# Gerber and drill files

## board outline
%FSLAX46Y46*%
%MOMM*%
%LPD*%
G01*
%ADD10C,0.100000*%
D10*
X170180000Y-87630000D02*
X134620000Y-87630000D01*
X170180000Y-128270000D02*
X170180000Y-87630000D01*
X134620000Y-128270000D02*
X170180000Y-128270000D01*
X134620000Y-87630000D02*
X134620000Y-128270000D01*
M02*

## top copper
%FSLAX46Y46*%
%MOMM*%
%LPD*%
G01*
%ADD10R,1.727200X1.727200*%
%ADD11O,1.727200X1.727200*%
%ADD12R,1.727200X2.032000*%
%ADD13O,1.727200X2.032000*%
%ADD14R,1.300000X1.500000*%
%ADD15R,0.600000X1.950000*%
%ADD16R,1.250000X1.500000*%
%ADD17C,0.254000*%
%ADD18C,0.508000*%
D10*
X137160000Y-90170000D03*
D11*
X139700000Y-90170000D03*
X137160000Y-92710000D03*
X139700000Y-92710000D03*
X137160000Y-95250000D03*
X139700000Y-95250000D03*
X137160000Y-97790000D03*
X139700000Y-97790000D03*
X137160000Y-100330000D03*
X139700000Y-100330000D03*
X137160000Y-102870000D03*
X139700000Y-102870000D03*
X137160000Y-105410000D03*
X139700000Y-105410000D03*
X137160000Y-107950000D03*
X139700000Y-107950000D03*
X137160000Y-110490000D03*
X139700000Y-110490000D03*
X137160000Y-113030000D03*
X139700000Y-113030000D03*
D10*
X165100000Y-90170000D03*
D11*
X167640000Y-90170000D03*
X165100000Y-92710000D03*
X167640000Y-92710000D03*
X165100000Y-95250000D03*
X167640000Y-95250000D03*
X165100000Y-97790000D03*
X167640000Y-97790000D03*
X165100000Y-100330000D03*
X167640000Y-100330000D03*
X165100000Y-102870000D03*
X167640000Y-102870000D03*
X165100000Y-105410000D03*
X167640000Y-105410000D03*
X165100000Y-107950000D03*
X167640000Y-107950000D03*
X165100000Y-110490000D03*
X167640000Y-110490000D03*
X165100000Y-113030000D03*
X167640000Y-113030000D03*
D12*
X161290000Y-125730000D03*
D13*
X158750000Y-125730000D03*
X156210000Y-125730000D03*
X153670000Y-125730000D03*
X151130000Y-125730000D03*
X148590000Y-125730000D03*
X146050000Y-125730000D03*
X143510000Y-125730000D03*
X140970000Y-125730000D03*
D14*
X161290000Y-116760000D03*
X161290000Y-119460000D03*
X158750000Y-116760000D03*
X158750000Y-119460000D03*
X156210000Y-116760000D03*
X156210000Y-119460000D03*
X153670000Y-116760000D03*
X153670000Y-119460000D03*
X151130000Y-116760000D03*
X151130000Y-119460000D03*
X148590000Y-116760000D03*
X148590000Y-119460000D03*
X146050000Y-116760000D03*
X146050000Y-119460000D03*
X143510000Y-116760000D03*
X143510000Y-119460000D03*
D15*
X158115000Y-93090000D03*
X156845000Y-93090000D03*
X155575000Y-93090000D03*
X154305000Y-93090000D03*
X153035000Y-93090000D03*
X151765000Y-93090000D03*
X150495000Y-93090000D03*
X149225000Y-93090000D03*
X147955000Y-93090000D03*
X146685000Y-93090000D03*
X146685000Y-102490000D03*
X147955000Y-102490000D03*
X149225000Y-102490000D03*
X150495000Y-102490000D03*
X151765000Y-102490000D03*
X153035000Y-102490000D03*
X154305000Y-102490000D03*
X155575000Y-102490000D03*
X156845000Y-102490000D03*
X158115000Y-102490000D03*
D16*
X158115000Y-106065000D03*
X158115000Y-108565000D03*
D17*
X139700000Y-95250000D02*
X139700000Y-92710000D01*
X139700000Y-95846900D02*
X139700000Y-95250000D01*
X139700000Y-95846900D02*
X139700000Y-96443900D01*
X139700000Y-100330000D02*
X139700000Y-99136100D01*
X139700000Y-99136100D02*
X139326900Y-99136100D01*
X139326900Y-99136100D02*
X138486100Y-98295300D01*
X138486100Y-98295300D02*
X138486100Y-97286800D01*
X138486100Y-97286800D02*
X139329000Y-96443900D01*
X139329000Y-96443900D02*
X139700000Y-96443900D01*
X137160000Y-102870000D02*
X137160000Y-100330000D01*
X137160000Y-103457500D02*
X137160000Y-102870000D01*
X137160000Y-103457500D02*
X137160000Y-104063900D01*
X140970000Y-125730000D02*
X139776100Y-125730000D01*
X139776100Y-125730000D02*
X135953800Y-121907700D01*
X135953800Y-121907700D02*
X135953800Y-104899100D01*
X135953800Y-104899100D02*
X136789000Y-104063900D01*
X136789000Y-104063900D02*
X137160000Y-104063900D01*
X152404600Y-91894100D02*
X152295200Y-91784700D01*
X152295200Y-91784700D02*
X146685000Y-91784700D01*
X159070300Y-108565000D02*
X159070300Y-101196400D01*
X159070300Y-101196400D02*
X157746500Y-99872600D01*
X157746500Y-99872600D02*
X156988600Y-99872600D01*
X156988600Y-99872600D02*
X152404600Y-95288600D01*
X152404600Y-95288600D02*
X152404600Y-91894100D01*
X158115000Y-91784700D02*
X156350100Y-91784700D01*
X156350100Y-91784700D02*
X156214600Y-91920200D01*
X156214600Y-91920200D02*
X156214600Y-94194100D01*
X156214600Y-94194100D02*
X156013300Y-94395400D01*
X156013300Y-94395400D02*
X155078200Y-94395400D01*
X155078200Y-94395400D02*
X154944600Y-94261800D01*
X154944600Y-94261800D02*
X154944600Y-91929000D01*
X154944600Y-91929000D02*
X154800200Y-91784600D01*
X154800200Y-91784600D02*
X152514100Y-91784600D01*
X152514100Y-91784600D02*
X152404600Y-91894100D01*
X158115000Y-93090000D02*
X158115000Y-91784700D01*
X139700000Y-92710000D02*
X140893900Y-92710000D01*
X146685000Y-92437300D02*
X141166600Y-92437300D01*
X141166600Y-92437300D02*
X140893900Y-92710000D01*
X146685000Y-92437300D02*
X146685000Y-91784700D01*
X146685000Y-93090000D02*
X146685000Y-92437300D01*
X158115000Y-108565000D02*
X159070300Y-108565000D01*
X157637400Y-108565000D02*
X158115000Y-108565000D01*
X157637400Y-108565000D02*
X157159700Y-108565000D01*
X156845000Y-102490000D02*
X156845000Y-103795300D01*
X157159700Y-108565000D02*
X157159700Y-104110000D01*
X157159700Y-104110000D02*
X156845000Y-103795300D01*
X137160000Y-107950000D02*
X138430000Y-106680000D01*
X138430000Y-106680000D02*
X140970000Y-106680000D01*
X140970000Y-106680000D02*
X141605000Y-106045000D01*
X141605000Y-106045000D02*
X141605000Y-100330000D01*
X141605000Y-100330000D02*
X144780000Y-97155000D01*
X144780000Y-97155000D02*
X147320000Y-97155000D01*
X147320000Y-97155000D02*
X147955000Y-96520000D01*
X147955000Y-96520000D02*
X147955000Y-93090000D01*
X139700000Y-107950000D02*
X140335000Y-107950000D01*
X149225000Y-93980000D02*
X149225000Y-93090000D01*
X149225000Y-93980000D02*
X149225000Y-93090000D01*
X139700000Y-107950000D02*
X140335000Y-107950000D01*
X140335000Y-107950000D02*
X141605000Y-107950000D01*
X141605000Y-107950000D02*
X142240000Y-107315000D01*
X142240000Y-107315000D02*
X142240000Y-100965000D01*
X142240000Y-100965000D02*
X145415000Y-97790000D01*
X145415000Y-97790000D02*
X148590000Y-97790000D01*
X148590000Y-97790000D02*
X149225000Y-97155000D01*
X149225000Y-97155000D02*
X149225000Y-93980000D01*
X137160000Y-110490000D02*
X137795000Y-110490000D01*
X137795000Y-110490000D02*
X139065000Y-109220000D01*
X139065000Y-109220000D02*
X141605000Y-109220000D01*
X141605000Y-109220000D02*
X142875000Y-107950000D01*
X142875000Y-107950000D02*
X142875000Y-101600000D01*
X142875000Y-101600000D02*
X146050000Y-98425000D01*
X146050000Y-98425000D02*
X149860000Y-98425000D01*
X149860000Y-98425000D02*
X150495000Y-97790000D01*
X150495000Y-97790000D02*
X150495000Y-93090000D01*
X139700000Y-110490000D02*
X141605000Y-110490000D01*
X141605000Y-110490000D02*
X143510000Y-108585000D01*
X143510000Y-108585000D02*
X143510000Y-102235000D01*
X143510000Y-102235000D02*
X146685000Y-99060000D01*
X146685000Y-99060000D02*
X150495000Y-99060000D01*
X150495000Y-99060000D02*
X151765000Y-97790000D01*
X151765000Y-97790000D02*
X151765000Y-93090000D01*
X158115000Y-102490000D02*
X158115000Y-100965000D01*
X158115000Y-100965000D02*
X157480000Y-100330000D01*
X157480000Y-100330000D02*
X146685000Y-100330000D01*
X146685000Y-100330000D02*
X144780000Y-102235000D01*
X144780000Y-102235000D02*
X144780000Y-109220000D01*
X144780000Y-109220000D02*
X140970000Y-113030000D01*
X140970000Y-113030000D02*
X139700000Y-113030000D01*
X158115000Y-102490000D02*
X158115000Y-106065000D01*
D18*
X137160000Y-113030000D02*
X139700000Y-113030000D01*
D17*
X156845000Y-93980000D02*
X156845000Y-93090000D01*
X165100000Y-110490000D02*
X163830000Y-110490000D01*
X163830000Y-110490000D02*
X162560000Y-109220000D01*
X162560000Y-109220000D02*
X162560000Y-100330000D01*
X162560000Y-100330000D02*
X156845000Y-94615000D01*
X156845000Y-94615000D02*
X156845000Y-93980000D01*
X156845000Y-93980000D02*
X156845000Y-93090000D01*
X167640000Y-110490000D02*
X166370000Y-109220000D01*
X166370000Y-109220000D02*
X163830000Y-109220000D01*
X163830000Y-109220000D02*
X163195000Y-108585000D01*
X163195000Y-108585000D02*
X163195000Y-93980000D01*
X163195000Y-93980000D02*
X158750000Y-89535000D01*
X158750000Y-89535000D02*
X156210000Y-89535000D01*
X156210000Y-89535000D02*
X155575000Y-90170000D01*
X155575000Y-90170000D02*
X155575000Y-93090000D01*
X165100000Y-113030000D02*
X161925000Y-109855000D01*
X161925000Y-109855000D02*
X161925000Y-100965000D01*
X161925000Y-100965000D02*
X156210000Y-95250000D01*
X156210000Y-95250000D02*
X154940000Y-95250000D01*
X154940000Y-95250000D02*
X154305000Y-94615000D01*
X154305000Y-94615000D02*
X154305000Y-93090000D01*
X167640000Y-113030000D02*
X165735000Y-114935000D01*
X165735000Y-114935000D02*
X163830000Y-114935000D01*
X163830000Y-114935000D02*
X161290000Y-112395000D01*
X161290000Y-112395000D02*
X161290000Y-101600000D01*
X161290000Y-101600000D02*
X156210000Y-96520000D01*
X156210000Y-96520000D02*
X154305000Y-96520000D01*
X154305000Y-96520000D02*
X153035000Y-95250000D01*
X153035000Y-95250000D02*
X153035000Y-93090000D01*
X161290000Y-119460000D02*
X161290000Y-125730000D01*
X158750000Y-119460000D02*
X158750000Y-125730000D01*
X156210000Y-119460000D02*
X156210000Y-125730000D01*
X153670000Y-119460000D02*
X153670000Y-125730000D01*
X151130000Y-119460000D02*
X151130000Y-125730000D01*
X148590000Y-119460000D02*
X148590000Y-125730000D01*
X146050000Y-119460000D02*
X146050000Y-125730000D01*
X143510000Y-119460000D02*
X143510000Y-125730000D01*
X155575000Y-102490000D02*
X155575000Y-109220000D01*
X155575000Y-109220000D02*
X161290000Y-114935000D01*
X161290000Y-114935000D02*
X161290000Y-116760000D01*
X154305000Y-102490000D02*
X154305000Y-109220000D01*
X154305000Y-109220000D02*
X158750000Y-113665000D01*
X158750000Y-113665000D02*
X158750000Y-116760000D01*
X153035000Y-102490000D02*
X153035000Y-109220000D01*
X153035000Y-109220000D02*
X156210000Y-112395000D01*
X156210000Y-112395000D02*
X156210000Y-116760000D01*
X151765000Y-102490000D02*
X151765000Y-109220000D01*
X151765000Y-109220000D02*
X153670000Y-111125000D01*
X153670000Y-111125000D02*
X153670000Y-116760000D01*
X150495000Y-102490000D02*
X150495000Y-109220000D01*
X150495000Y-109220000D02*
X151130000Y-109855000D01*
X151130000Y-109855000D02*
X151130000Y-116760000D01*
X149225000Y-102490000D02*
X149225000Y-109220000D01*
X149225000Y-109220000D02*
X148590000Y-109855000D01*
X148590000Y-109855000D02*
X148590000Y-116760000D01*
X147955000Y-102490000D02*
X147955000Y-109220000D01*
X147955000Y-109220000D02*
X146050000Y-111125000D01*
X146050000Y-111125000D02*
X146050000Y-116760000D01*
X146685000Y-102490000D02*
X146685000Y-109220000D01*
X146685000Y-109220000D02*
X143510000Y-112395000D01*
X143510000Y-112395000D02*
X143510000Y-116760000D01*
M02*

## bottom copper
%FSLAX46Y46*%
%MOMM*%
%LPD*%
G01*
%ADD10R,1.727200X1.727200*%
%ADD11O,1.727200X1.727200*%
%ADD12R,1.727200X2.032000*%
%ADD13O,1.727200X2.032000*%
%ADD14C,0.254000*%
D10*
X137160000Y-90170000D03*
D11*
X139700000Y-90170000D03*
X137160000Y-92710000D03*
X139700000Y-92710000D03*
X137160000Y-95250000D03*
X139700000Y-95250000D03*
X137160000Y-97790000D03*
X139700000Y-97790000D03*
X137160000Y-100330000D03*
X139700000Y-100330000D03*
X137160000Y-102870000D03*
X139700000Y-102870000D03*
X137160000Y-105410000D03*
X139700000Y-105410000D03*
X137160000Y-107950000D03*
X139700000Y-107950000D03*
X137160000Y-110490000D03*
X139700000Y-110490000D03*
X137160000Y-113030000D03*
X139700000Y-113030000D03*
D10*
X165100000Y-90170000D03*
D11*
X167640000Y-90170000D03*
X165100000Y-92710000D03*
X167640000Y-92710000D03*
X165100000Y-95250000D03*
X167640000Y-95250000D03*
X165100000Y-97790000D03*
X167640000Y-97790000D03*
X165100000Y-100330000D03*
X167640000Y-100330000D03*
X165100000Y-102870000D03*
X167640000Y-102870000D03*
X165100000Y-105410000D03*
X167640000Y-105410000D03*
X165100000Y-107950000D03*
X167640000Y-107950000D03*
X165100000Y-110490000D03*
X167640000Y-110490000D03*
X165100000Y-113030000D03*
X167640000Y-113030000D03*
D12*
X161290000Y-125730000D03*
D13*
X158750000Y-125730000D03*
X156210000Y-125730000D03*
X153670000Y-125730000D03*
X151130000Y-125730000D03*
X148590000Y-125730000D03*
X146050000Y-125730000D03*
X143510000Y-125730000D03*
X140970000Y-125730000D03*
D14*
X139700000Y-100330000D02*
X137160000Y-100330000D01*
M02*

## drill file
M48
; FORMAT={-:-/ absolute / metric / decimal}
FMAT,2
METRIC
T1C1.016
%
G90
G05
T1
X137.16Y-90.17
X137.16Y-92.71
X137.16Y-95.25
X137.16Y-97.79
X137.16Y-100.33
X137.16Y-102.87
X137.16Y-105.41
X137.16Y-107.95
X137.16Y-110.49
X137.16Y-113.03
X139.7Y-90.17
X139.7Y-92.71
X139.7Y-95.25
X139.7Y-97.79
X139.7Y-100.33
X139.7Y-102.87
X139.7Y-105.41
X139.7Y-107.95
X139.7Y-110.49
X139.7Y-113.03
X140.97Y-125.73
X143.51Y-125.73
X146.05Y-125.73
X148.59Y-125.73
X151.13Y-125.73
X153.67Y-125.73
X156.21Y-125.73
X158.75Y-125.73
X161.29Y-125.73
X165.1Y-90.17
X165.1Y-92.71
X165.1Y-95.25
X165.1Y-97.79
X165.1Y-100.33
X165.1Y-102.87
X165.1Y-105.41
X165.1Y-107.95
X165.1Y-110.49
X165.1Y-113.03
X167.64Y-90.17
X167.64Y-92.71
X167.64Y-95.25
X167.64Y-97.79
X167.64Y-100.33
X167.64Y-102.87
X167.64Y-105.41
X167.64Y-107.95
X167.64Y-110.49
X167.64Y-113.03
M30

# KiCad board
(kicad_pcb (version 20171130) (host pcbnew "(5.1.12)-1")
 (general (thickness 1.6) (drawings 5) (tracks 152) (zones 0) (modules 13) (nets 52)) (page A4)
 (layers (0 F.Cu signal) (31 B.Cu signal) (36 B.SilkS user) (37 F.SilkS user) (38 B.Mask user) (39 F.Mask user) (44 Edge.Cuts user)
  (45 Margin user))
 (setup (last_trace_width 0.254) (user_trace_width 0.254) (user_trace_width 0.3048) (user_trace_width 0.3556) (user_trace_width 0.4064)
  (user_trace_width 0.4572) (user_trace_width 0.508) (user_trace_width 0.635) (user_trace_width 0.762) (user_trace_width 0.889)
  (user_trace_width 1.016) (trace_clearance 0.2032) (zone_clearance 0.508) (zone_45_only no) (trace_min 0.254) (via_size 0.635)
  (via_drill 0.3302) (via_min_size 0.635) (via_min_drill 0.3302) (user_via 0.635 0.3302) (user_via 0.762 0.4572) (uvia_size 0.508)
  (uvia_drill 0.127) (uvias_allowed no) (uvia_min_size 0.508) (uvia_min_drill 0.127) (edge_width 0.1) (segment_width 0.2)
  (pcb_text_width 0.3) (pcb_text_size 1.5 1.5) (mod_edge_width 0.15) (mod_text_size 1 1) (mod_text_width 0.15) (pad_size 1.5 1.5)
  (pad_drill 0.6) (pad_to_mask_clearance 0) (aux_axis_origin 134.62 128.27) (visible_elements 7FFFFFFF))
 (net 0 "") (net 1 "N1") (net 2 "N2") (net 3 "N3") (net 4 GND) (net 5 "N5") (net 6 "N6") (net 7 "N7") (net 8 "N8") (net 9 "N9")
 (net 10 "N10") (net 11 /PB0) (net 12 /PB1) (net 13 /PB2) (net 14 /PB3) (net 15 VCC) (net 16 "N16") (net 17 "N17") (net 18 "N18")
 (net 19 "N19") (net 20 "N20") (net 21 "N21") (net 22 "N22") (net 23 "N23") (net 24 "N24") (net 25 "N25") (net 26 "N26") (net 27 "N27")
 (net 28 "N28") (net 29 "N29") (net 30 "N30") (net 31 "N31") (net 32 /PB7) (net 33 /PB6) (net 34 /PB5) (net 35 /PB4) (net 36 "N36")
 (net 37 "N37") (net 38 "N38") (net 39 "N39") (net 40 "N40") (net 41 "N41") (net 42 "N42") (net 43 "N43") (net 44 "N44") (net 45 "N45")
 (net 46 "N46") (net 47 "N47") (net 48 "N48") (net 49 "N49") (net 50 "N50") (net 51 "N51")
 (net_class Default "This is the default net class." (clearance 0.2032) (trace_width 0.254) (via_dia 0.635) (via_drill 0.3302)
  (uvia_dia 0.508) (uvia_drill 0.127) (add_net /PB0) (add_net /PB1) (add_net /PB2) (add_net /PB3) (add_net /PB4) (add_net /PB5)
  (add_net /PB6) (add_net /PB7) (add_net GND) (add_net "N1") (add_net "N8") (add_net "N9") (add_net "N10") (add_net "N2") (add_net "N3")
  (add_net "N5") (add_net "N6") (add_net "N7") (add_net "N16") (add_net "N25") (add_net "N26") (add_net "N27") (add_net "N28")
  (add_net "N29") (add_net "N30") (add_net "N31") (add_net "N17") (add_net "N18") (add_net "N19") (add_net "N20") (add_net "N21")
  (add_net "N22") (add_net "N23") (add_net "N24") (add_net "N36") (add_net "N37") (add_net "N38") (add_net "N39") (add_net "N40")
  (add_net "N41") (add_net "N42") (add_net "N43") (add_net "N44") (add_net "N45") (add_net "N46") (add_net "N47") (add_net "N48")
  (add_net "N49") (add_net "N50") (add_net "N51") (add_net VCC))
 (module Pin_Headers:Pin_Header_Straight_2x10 (layer F.Cu) (at 137.16 90.17)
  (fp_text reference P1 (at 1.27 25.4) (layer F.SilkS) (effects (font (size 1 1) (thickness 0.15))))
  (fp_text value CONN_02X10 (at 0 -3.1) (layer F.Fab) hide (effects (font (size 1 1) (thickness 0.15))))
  (pad 1 thru_hole rect (at 0 0) (size 1.7272 1.7272) (drill 1.016) (layers *.Cu *.Mask F.SilkS) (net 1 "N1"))
  (pad 2 thru_hole oval (at 2.54 0) (size 1.7272 1.7272) (drill 1.016) (layers *.Cu *.Mask F.SilkS) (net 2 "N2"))
  (pad 3 thru_hole oval (at 0 2.54) (size 1.7272 1.7272) (drill 1.016) (layers *.Cu *.Mask F.SilkS) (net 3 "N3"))
  (pad 4 thru_hole oval (at 2.54 2.54) (size 1.7272 1.7272) (drill 1.016) (layers *.Cu *.Mask F.SilkS) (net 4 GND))
  (pad 5 thru_hole oval (at 0 5.08) (size 1.7272 1.7272) (drill 1.016) (layers *.Cu *.Mask F.SilkS) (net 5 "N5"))
  (pad 6 thru_hole oval (at 2.54 5.08) (size 1.7272 1.7272) (drill 1.016) (layers *.Cu *.Mask F.SilkS) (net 4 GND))
  (pad 7 thru_hole oval (at 0 7.62) (size 1.7272 1.7272) (drill 1.016) (layers *.Cu *.Mask F.SilkS) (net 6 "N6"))
  (pad 8 thru_hole oval (at 2.54 7.62) (size 1.7272 1.7272) (drill 1.016) (layers *.Cu *.Mask F.SilkS) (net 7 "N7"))
  (pad 9 thru_hole oval (at 0 10.16) (size 1.7272 1.7272) (drill 1.016) (layers *.Cu *.Mask F.SilkS) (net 4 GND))
  (pad 10 thru_hole oval (at 2.54 10.16) (size 1.7272 1.7272) (drill 1.016) (layers *.Cu *.Mask F.SilkS) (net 4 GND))
  (pad 11 thru_hole oval (at 0 12.7) (size 1.7272 1.7272) (drill 1.016) (layers *.Cu *.Mask F.SilkS) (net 4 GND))
  (pad 12 thru_hole oval (at 2.54 12.7) (size 1.7272 1.7272) (drill 1.016) (layers *.Cu *.Mask F.SilkS) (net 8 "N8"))
  (pad 13 thru_hole oval (at 0 15.24) (size 1.7272 1.7272) (drill 1.016) (layers *.Cu *.Mask F.SilkS) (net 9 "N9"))
  (pad 14 thru_hole oval (at 2.54 15.24) (size 1.7272 1.7272) (drill 1.016) (layers *.Cu *.Mask F.SilkS) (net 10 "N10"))
  (pad 15 thru_hole oval (at 0 17.78) (size 1.7272 1.7272) (drill 1.016) (layers *.Cu *.Mask F.SilkS) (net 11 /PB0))
  (pad 16 thru_hole oval (at 2.54 17.78) (size 1.7272 1.7272) (drill 1.016) (layers *.Cu *.Mask F.SilkS) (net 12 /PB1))
  (pad 17 thru_hole oval (at 0 20.32) (size 1.7272 1.7272) (drill 1.016) (layers *.Cu *.Mask F.SilkS) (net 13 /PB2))
  (pad 18 thru_hole oval (at 2.54 20.32) (size 1.7272 1.7272) (drill 1.016) (layers *.Cu *.Mask F.SilkS) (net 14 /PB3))
  (pad 19 thru_hole oval (at 0 22.86) (size 1.7272 1.7272) (drill 1.016) (layers *.Cu *.Mask F.SilkS) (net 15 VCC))
  (pad 20 thru_hole oval (at 2.54 22.86) (size 1.7272 1.7272) (drill 1.016) (layers *.Cu *.Mask F.SilkS) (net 15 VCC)))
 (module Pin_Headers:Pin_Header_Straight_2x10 (layer F.Cu) (at 165.1 90.17)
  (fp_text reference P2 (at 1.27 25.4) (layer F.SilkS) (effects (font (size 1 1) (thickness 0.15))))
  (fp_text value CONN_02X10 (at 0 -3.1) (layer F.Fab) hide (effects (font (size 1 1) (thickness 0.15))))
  (pad 1 thru_hole rect (at 0 0) (size 1.7272 1.7272) (drill 1.016) (layers *.Cu *.Mask F.SilkS) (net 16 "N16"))
  (pad 2 thru_hole oval (at 2.54 0) (size 1.7272 1.7272) (drill 1.016) (layers *.Cu *.Mask F.SilkS) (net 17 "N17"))
  (pad 3 thru_hole oval (at 0 2.54) (size 1.7272 1.7272) (drill 1.016) (layers *.Cu *.Mask F.SilkS) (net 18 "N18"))
  (pad 4 thru_hole oval (at 2.54 2.54) (size 1.7272 1.7272) (drill 1.016) (layers *.Cu *.Mask F.SilkS) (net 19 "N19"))
  (pad 5 thru_hole oval (at 0 5.08) (size 1.7272 1.7272) (drill 1.016) (layers *.Cu *.Mask F.SilkS) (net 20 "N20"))
  (pad 6 thru_hole oval (at 2.54 5.08) (size 1.7272 1.7272) (drill 1.016) (layers *.Cu *.Mask F.SilkS) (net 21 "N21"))
  (pad 7 thru_hole oval (at 0 7.62) (size 1.7272 1.7272) (drill 1.016) (layers *.Cu *.Mask F.SilkS) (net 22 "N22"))
  (pad 8 thru_hole oval (at 2.54 7.62) (size 1.7272 1.7272) (drill 1.016) (layers *.Cu *.Mask F.SilkS) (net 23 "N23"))
  (pad 9 thru_hole oval (at 0 10.16) (size 1.7272 1.7272) (drill 1.016) (layers *.Cu *.Mask F.SilkS) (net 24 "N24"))
  (pad 10 thru_hole oval (at 2.54 10.16) (size 1.7272 1.7272) (drill 1.016) (layers *.Cu *.Mask F.SilkS) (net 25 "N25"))
  (pad 11 thru_hole oval (at 0 12.7) (size 1.7272 1.7272) (drill 1.016) (layers *.Cu *.Mask F.SilkS) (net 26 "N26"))
  (pad 12 thru_hole oval (at 2.54 12.7) (size 1.7272 1.7272) (drill 1.016) (layers *.Cu *.Mask F.SilkS) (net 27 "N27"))
  (pad 13 thru_hole oval (at 0 15.24) (size 1.7272 1.7272) (drill 1.016) (layers *.Cu *.Mask F.SilkS) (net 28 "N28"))
  (pad 14 thru_hole oval (at 2.54 15.24) (size 1.7272 1.7272) (drill 1.016) (layers *.Cu *.Mask F.SilkS) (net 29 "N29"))
  (pad 15 thru_hole oval (at 0 17.78) (size 1.7272 1.7272) (drill 1.016) (layers *.Cu *.Mask F.SilkS) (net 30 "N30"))
  (pad 16 thru_hole oval (at 2.54 17.78) (size 1.7272 1.7272) (drill 1.016) (layers *.Cu *.Mask F.SilkS) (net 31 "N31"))
  (pad 17 thru_hole oval (at 0 20.32) (size 1.7272 1.7272) (drill 1.016) (layers *.Cu *.Mask F.SilkS) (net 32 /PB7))
  (pad 18 thru_hole oval (at 2.54 20.32) (size 1.7272 1.7272) (drill 1.016) (layers *.Cu *.Mask F.SilkS) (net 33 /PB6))
  (pad 19 thru_hole oval (at 0 22.86) (size 1.7272 1.7272) (drill 1.016) (layers *.Cu *.Mask F.SilkS) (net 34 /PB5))
  (pad 20 thru_hole oval (at 2.54 22.86) (size 1.7272 1.7272) (drill 1.016) (layers *.Cu *.Mask F.SilkS) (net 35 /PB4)))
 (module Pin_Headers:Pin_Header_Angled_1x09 (layer F.Cu) (at 161.29 125.73 270)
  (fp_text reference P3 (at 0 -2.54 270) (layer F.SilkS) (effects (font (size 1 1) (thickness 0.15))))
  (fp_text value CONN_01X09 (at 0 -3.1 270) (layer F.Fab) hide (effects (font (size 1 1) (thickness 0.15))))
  (pad 1 thru_hole rect (at 0 0 270) (size 2.032 1.7272) (drill 1.016) (layers *.Cu *.Mask F.SilkS) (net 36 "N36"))
  (pad 2 thru_hole oval (at 0 2.54 270) (size 2.032 1.7272) (drill 1.016) (layers *.Cu *.Mask F.SilkS) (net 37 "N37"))
  (pad 3 thru_hole oval (at 0 5.08 270) (size 2.032 1.7272) (drill 1.016) (layers *.Cu *.Mask F.SilkS) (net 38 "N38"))
  (pad 4 thru_hole oval (at 0 7.62 270) (size 2.032 1.7272) (drill 1.016) (layers *.Cu *.Mask F.SilkS) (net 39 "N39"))
  (pad 5 thru_hole oval (at 0 10.16 270) (size 2.032 1.7272) (drill 1.016) (layers *.Cu *.Mask F.SilkS) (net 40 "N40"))
  (pad 6 thru_hole oval (at 0 12.7 270) (size 2.032 1.7272) (drill 1.016) (layers *.Cu *.Mask F.SilkS) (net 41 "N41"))
  (pad 7 thru_hole oval (at 0 15.24 270) (size 2.032 1.7272) (drill 1.016) (layers *.Cu *.Mask F.SilkS) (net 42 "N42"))
  (pad 8 thru_hole oval (at 0 17.78 270) (size 2.032 1.7272) (drill 1.016) (layers *.Cu *.Mask F.SilkS) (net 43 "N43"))
  (pad 9 thru_hole oval (at 0 20.32 270) (size 2.032 1.7272) (drill 1.016) (layers *.Cu *.Mask F.SilkS) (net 4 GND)))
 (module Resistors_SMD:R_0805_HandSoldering (layer F.Cu) (at 161.29 118.11 270)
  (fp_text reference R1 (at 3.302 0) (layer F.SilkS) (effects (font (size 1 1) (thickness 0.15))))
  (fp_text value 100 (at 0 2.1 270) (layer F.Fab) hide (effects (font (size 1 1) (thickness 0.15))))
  (pad 1 smd rect (at -1.35 0 270) (size 1.5 1.3) (layers F.Cu F.Mask) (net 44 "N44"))
  (pad 2 smd rect (at 1.35 0 270) (size 1.5 1.3) (layers F.Cu F.Mask) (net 36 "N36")))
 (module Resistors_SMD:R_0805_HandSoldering (layer F.Cu) (at 158.75 118.11 270)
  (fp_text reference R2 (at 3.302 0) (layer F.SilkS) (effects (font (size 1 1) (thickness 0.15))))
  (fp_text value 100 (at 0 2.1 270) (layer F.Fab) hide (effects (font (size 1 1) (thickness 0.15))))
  (pad 1 smd rect (at -1.35 0 270) (size 1.5 1.3) (layers F.Cu F.Mask) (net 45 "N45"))
  (pad 2 smd rect (at 1.35 0 270) (size 1.5 1.3) (layers F.Cu F.Mask) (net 37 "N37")))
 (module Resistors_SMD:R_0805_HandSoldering (layer F.Cu) (at 156.21 118.11 270)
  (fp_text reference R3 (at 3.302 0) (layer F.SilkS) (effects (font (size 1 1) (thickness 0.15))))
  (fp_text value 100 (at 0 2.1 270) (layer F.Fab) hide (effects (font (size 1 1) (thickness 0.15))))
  (pad 1 smd rect (at -1.35 0 270) (size 1.5 1.3) (layers F.Cu F.Mask) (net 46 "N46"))
  (pad 2 smd rect (at 1.35 0 270) (size 1.5 1.3) (layers F.Cu F.Mask) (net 38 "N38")))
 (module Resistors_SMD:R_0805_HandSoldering (layer F.Cu) (at 153.67 118.11 270)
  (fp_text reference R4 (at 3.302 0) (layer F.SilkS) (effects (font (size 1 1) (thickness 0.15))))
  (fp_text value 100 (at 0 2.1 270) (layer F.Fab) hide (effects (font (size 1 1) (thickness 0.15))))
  (pad 1 smd rect (at -1.35 0 270) (size 1.5 1.3) (layers F.Cu F.Mask) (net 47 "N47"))
  (pad 2 smd rect (at 1.35 0 270) (size 1.5 1.3) (layers F.Cu F.Mask) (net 39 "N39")))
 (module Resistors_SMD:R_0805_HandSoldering (layer F.Cu) (at 151.13 118.11 270)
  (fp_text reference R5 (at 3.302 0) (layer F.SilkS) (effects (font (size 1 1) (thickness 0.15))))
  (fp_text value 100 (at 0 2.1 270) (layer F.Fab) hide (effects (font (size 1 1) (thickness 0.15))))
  (pad 1 smd rect (at -1.35 0 270) (size 1.5 1.3) (layers F.Cu F.Mask) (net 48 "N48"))
  (pad 2 smd rect (at 1.35 0 270) (size 1.5 1.3) (layers F.Cu F.Mask) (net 40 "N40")))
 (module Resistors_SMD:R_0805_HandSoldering (layer F.Cu) (at 148.59 118.11 270)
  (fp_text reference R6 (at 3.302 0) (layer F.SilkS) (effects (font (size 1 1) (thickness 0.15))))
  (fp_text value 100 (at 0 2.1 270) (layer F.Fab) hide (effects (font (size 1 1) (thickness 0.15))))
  (pad 1 smd rect (at -1.35 0 270) (size 1.5 1.3) (layers F.Cu F.Mask) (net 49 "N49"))
  (pad 2 smd rect (at 1.35 0 270) (size 1.5 1.3) (layers F.Cu F.Mask) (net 41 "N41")))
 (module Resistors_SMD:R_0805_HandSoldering (layer F.Cu) (at 146.05 118.11 270)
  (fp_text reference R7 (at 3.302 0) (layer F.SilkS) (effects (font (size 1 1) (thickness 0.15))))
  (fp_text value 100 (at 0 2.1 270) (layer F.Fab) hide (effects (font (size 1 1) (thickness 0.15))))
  (pad 1 smd rect (at -1.35 0 270) (size 1.5 1.3) (layers F.Cu F.Mask) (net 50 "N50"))
  (pad 2 smd rect (at 1.35 0 270) (size 1.5 1.3) (layers F.Cu F.Mask) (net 42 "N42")))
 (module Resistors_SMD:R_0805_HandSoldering (layer F.Cu) (at 143.51 118.11 270)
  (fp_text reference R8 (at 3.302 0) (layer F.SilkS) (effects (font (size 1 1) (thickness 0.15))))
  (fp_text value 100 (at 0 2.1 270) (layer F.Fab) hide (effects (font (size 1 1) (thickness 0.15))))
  (pad 1 smd rect (at -1.35 0 270) (size 1.5 1.3) (layers F.Cu F.Mask) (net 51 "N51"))
  (pad 2 smd rect (at 1.35 0 270) (size 1.5 1.3) (layers F.Cu F.Mask) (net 43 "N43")))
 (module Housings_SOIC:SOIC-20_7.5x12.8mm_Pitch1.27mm (layer F.Cu) (at 152.4 97.79 270)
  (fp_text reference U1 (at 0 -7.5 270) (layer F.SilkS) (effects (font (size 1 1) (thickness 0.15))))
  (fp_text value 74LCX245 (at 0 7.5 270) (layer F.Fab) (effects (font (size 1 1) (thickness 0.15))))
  (pad 1 smd rect (at -4.7 -5.715 270) (size 1.95 0.6) (layers F.Cu F.Mask) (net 4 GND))
  (pad 2 smd rect (at -4.7 -4.445 270) (size 1.95 0.6) (layers F.Cu F.Mask) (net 32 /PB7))
  (pad 3 smd rect (at -4.7 -3.175 270) (size 1.95 0.6) (layers F.Cu F.Mask) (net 33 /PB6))
  (pad 4 smd rect (at -4.7 -1.905 270) (size 1.95 0.6) (layers F.Cu F.Mask) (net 34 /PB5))
  (pad 5 smd rect (at -4.7 -0.635 270) (size 1.95 0.6) (layers F.Cu F.Mask) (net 35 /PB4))
  (pad 6 smd rect (at -4.7 0.635 270) (size 1.95 0.6) (layers F.Cu F.Mask) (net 14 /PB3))
  (pad 7 smd rect (at -4.7 1.905 270) (size 1.95 0.6) (layers F.Cu F.Mask) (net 13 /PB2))
  (pad 8 smd rect (at -4.7 3.175 270) (size 1.95 0.6) (layers F.Cu F.Mask) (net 12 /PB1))
  (pad 9 smd rect (at -4.7 4.445 270) (size 1.95 0.6) (layers F.Cu F.Mask) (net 11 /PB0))
  (pad 10 smd rect (at -4.7 5.715 270) (size 1.95 0.6) (layers F.Cu F.Mask) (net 4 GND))
  (pad 11 smd rect (at 4.7 5.715 270) (size 1.95 0.6) (layers F.Cu F.Mask) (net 51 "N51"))
  (pad 12 smd rect (at 4.7 4.445 270) (size 1.95 0.6) (layers F.Cu F.Mask) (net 50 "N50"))
  (pad 13 smd rect (at 4.7 3.175 270) (size 1.95 0.6) (layers F.Cu F.Mask) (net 49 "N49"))
  (pad 14 smd rect (at 4.7 1.905 270) (size 1.95 0.6) (layers F.Cu F.Mask) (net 48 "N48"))
  (pad 15 smd rect (at 4.7 0.635 270) (size 1.95 0.6) (layers F.Cu F.Mask) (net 47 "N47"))
  (pad 16 smd rect (at 4.7 -0.635 270) (size 1.95 0.6) (layers F.Cu F.Mask) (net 46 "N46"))
  (pad 17 smd rect (at 4.7 -1.905 270) (size 1.95 0.6) (layers F.Cu F.Mask) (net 45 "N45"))
  (pad 18 smd rect (at 4.7 -3.175 270) (size 1.95 0.6) (layers F.Cu F.Mask) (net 44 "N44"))
  (pad 19 smd rect (at 4.7 -4.445 270) (size 1.95 0.6) (layers F.Cu F.Mask) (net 4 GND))
  (pad 20 smd rect (at 4.7 -5.715 270) (size 1.95 0.6) (layers F.Cu F.Mask) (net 15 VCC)))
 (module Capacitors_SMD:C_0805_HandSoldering (layer F.Cu) (at 158.115 107.315 270)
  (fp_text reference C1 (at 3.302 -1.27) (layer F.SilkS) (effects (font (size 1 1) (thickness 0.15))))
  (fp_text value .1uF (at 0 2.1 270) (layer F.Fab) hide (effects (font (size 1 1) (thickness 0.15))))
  (pad 1 smd rect (at -1.25 0 270) (size 1.5 1.25) (layers F.Cu F.Mask) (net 15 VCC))
  (pad 2 smd rect (at 1.25 0 270) (size 1.5 1.25) (layers F.Cu F.Mask) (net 4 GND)))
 (gr_line (start 170.18 87.63) (end 134.62 87.63) (angle 90) (layer Edge.Cuts) (width 0.1))
 (gr_line (start 170.18 128.27) (end 170.18 87.63) (angle 90) (layer Edge.Cuts) (width 0.1))
 (gr_line (start 134.62 128.27) (end 170.18 128.27) (angle 90) (layer Edge.Cuts) (width 0.1))
 (gr_line (start 134.62 87.63) (end 134.62 128.27) (angle 90) (layer Edge.Cuts) (width 0.1))
 (segment (start 139.7 95.25) (end 139.7 92.71) (width 0.254) (layer F.Cu) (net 4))
 (segment (start 139.7 95.8469) (end 139.7 95.25) (width 0.254) (layer F.Cu) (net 4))
 (segment (start 139.7 95.8469) (end 139.7 96.4439) (width 0.254) (layer F.Cu) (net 4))
 (segment (start 139.7 100.33) (end 139.7 99.1361) (width 0.254) (layer F.Cu) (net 4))
 (segment (start 139.7 99.1361) (end 139.3269 99.1361) (width 0.254) (layer F.Cu) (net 4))
 (segment (start 139.3269 99.1361) (end 138.4861 98.2953) (width 0.254) (layer F.Cu) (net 4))
 (segment (start 138.4861 98.2953) (end 138.4861 97.2868) (width 0.254) (layer F.Cu) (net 4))
 (segment (start 138.4861 97.2868) (end 139.329 96.4439) (width 0.254) (layer F.Cu) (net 4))
 (segment (start 139.329 96.4439) (end 139.7 96.4439) (width 0.254) (layer F.Cu) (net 4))
 (segment (start 139.7 100.33) (end 137.16 100.33) (width 0.254) (layer B.Cu) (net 4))
 (segment (start 137.16 102.87) (end 137.16 100.33) (width 0.254) (layer F.Cu) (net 4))
 (segment (start 137.16 103.4575) (end 137.16 102.87) (width 0.254) (layer F.Cu) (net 4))
 (segment (start 137.16 103.4575) (end 137.16 104.0639) (width 0.254) (layer F.Cu) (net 4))
 (segment (start 140.97 125.73) (end 139.7761 125.73) (width 0.254) (layer F.Cu) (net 4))
 (segment (start 139.7761 125.73) (end 135.9538 121.9077) (width 0.254) (layer F.Cu) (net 4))
 (segment (start 135.9538 121.9077) (end 135.9538 104.8991) (width 0.254) (layer F.Cu) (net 4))
 (segment (start 135.9538 104.8991) (end 136.789 104.0639) (width 0.254) (layer F.Cu) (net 4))
 (segment (start 136.789 104.0639) (end 137.16 104.0639) (width 0.254) (layer F.Cu) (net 4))
 (segment (start 152.4046 91.8941) (end 152.2952 91.7847) (width 0.254) (layer F.Cu) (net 4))
 (segment (start 152.2952 91.7847) (end 146.685 91.7847) (width 0.254) (layer F.Cu) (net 4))
 (segment (start 159.0703 108.565) (end 159.0703 101.1964) (width 0.254) (layer F.Cu) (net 4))
 (segment (start 159.0703 101.1964) (end 157.7465 99.8726) (width 0.254) (layer F.Cu) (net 4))
 (segment (start 157.7465 99.8726) (end 156.9886 99.8726) (width 0.254) (layer F.Cu) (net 4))
 (segment (start 156.9886 99.8726) (end 152.4046 95.2886) (width 0.254) (layer F.Cu) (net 4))
 (segment (start 152.4046 95.2886) (end 152.4046 91.8941) (width 0.254) (layer F.Cu) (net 4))
 (segment (start 158.115 91.7847) (end 156.3501 91.7847) (width 0.254) (layer F.Cu) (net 4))
 (segment (start 156.3501 91.7847) (end 156.2146 91.9202) (width 0.254) (layer F.Cu) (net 4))
 (segment (start 156.2146 91.9202) (end 156.2146 94.1941) (width 0.254) (layer F.Cu) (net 4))
 (segment (start 156.2146 94.1941) (end 156.0133 94.3954) (width 0.254) (layer F.Cu) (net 4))
 (segment (start 156.0133 94.3954) (end 155.0782 94.3954) (width 0.254) (layer F.Cu) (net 4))
 (segment (start 155.0782 94.3954) (end 154.9446 94.2618) (width 0.254) (layer F.Cu) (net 4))
 (segment (start 154.9446 94.2618) (end 154.9446 91.929) (width 0.254) (layer F.Cu) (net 4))
 (segment (start 154.9446 91.929) (end 154.8002 91.7846) (width 0.254) (layer F.Cu) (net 4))
 (segment (start 154.8002 91.7846) (end 152.5141 91.7846) (width 0.254) (layer F.Cu) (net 4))
 (segment (start 152.5141 91.7846) (end 152.4046 91.8941) (width 0.254) (layer F.Cu) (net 4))
 (segment (start 158.115 93.09) (end 158.115 91.7847) (width 0.254) (layer F.Cu) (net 4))
 (segment (start 139.7 92.71) (end 140.8939 92.71) (width 0.254) (layer F.Cu) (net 4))
 (segment (start 146.685 92.4373) (end 141.1666 92.4373) (width 0.254) (layer F.Cu) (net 4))
 (segment (start 141.1666 92.4373) (end 140.8939 92.71) (width 0.254) (layer F.Cu) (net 4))
 (segment (start 146.685 92.4373) (end 146.685 91.7847) (width 0.254) (layer F.Cu) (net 4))
 (segment (start 146.685 93.09) (end 146.685 92.4373) (width 0.254) (layer F.Cu) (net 4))
 (segment (start 158.115 108.565) (end 159.0703 108.565) (width 0.254) (layer F.Cu) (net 4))
 (segment (start 157.6374 108.565) (end 158.115 108.565) (width 0.254) (layer F.Cu) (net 4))
 (segment (start 157.6374 108.565) (end 157.1597 108.565) (width 0.254) (layer F.Cu) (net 4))
 (segment (start 156.845 102.49) (end 156.845 103.7953) (width 0.254) (layer F.Cu) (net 4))
 (segment (start 157.1597 108.565) (end 157.1597 104.11) (width 0.254) (layer F.Cu) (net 4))
 (segment (start 157.1597 104.11) (end 156.845 103.7953) (width 0.254) (layer F.Cu) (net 4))
 (segment (start 137.16 107.95) (end 138.43 106.68) (width 0.254) (layer F.Cu) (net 11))
 (segment (start 138.43 106.68) (end 140.97 106.68) (width 0.254) (layer F.Cu) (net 11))
 (segment (start 140.97 106.68) (end 141.605 106.045) (width 0.254) (layer F.Cu) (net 11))
 (segment (start 141.605 106.045) (end 141.605 100.33) (width 0.254) (layer F.Cu) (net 11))
 (segment (start 141.605 100.33) (end 144.78 97.155) (width 0.254) (layer F.Cu) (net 11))
 (segment (start 144.78 97.155) (end 147.32 97.155) (width 0.254) (layer F.Cu) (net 11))
 (segment (start 147.32 97.155) (end 147.955 96.52) (width 0.254) (layer F.Cu) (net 11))
 (segment (start 147.955 96.52) (end 147.955 93.09) (width 0.254) (layer F.Cu) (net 11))
 (segment (start 139.7 107.95) (end 140.335 107.95) (width 0.254) (layer F.Cu) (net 12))
 (segment (start 149.225 93.98) (end 149.225 93.09) (width 0.254) (layer F.Cu) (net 12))
 (segment (start 149.225 93.98) (end 149.225 93.09) (width 0.254) (layer F.Cu) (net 12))
 (segment (start 139.7 107.95) (end 140.335 107.95) (width 0.254) (layer F.Cu) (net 12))
 (segment (start 140.335 107.95) (end 141.605 107.95) (width 0.254) (layer F.Cu) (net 12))
 (segment (start 141.605 107.95) (end 142.24 107.315) (width 0.254) (layer F.Cu) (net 12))
 (segment (start 142.24 107.315) (end 142.24 100.965) (width 0.254) (layer F.Cu) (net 12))
 (segment (start 142.24 100.965) (end 145.415 97.79) (width 0.254) (layer F.Cu) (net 12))
 (segment (start 145.415 97.79) (end 148.59 97.79) (width 0.254) (layer F.Cu) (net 12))
 (segment (start 148.59 97.79) (end 149.225 97.155) (width 0.254) (layer F.Cu) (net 12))
 (segment (start 149.225 97.155) (end 149.225 93.98) (width 0.254) (layer F.Cu) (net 12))
 (segment (start 137.16 110.49) (end 137.795 110.49) (width 0.254) (layer F.Cu) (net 13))
 (segment (start 137.795 110.49) (end 139.065 109.22) (width 0.254) (layer F.Cu) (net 13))
 (segment (start 139.065 109.22) (end 141.605 109.22) (width 0.254) (layer F.Cu) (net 13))
 (segment (start 141.605 109.22) (end 142.875 107.95) (width 0.254) (layer F.Cu) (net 13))
 (segment (start 142.875 107.95) (end 142.875 101.6) (width 0.254) (layer F.Cu) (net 13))
 (segment (start 142.875 101.6) (end 146.05 98.425) (width 0.254) (layer F.Cu) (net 13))
 (segment (start 146.05 98.425) (end 149.86 98.425) (width 0.254) (layer F.Cu) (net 13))
 (segment (start 149.86 98.425) (end 150.495 97.79) (width 0.254) (layer F.Cu) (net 13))
 (segment (start 150.495 97.79) (end 150.495 93.09) (width 0.254) (layer F.Cu) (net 13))
 (segment (start 139.7 110.49) (end 141.605 110.49) (width 0.254) (layer F.Cu) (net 14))
 (segment (start 141.605 110.49) (end 143.51 108.585) (width 0.254) (layer F.Cu) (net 14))
 (segment (start 143.51 108.585) (end 143.51 102.235) (width 0.254) (layer F.Cu) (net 14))
 (segment (start 143.51 102.235) (end 146.685 99.06) (width 0.254) (layer F.Cu) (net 14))
 (segment (start 146.685 99.06) (end 150.495 99.06) (width 0.254) (layer F.Cu) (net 14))
 (segment (start 150.495 99.06) (end 151.765 97.79) (width 0.254) (layer F.Cu) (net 14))
 (segment (start 151.765 97.79) (end 151.765 93.09) (width 0.254) (layer F.Cu) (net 14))
 (segment (start 158.115 102.49) (end 158.115 100.965) (width 0.254) (layer F.Cu) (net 15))
 (segment (start 158.115 100.965) (end 157.48 100.33) (width 0.254) (layer F.Cu) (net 15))
 (segment (start 157.48 100.33) (end 146.685 100.33) (width 0.254) (layer F.Cu) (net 15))
 (segment (start 146.685 100.33) (end 144.78 102.235) (width 0.254) (layer F.Cu) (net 15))
 (segment (start 144.78 102.235) (end 144.78 109.22) (width 0.254) (layer F.Cu) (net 15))
 (segment (start 144.78 109.22) (end 140.97 113.03) (width 0.254) (layer F.Cu) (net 15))
 (segment (start 140.97 113.03) (end 139.7 113.03) (width 0.254) (layer F.Cu) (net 15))
 (segment (start 158.115 102.49) (end 158.115 106.065) (width 0.254) (layer F.Cu) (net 15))
 (segment (start 137.16 113.03) (end 139.7 113.03) (width 0.508) (layer F.Cu) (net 15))
 (segment (start 156.845 93.98) (end 156.845 93.09) (width 0.254) (layer F.Cu) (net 32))
 (segment (start 165.1 110.49) (end 163.83 110.49) (width 0.254) (layer F.Cu) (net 32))
 (segment (start 163.83 110.49) (end 162.56 109.22) (width 0.254) (layer F.Cu) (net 32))
 (segment (start 162.56 109.22) (end 162.56 100.33) (width 0.254) (layer F.Cu) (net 32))
 (segment (start 162.56 100.33) (end 156.845 94.615) (width 0.254) (layer F.Cu) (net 32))
 (segment (start 156.845 94.615) (end 156.845 93.98) (width 0.254) (layer F.Cu) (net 32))
 (segment (start 156.845 93.98) (end 156.845 93.09) (width 0.254) (layer F.Cu) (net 32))
 (segment (start 167.64 110.49) (end 166.37 109.22) (width 0.254) (layer F.Cu) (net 33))
 (segment (start 166.37 109.22) (end 163.83 109.22) (width 0.254) (layer F.Cu) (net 33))
 (segment (start 163.83 109.22) (end 163.195 108.585) (width 0.254) (layer F.Cu) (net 33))
 (segment (start 163.195 108.585) (end 163.195 93.98) (width 0.254) (layer F.Cu) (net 33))
 (segment (start 163.195 93.98) (end 158.75 89.535) (width 0.254) (layer F.Cu) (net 33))
 (segment (start 158.75 89.535) (end 156.21 89.535) (width 0.254) (layer F.Cu) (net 33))
 (segment (start 156.21 89.535) (end 155.575 90.17) (width 0.254) (layer F.Cu) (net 33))
 (segment (start 155.575 90.17) (end 155.575 93.09) (width 0.254) (layer F.Cu) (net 33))
 (segment (start 165.1 113.03) (end 161.925 109.855) (width 0.254) (layer F.Cu) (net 34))
 (segment (start 161.925 109.855) (end 161.925 100.965) (width 0.254) (layer F.Cu) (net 34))
 (segment (start 161.925 100.965) (end 156.21 95.25) (width 0.254) (layer F.Cu) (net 34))
 (segment (start 156.21 95.25) (end 154.94 95.25) (width 0.254) (layer F.Cu) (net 34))
 (segment (start 154.94 95.25) (end 154.305 94.615) (width 0.254) (layer F.Cu) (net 34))
 (segment (start 154.305 94.615) (end 154.305 93.09) (width 0.254) (layer F.Cu) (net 34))
 (segment (start 167.64 113.03) (end 165.735 114.935) (width 0.254) (layer F.Cu) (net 35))
 (segment (start 165.735 114.935) (end 163.83 114.935) (width 0.254) (layer F.Cu) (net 35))
 (segment (start 163.83 114.935) (end 161.29 112.395) (width 0.254) (layer F.Cu) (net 35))
 (segment (start 161.29 112.395) (end 161.29 101.6) (width 0.254) (layer F.Cu) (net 35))
 (segment (start 161.29 101.6) (end 156.21 96.52) (width 0.254) (layer F.Cu) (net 35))
 (segment (start 156.21 96.52) (end 154.305 96.52) (width 0.254) (layer F.Cu) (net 35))
 (segment (start 154.305 96.52) (end 153.035 95.25) (width 0.254) (layer F.Cu) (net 35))
 (segment (start 153.035 95.25) (end 153.035 93.09) (width 0.254) (layer F.Cu) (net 35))
 (segment (start 161.29 119.46) (end 161.29 125.73) (width 0.254) (layer F.Cu) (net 36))
 (segment (start 158.75 119.46) (end 158.75 125.73) (width 0.254) (layer F.Cu) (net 37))
 (segment (start 156.21 119.46) (end 156.21 125.73) (width 0.254) (layer F.Cu) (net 38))
 (segment (start 153.67 119.46) (end 153.67 125.73) (width 0.254) (layer F.Cu) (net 39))
 (segment (start 151.13 119.46) (end 151.13 125.73) (width 0.254) (layer F.Cu) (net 40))
 (segment (start 148.59 119.46) (end 148.59 125.73) (width 0.254) (layer F.Cu) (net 41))
 (segment (start 146.05 119.46) (end 146.05 125.73) (width 0.254) (layer F.Cu) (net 42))
 (segment (start 143.51 119.46) (end 143.51 125.73) (width 0.254) (layer F.Cu) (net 43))
 (segment (start 155.575 102.49) (end 155.575 109.22) (width 0.254) (layer F.Cu) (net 44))
 (segment (start 155.575 109.22) (end 161.29 114.935) (width 0.254) (layer F.Cu) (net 44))
 (segment (start 161.29 114.935) (end 161.29 116.76) (width 0.254) (layer F.Cu) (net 44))
 (segment (start 154.305 102.49) (end 154.305 109.22) (width 0.254) (layer F.Cu) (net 45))
 (segment (start 154.305 109.22) (end 158.75 113.665) (width 0.254) (layer F.Cu) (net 45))
 (segment (start 158.75 113.665) (end 158.75 116.76) (width 0.254) (layer F.Cu) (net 45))
 (segment (start 153.035 102.49) (end 153.035 109.22) (width 0.254) (layer F.Cu) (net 46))
 (segment (start 153.035 109.22) (end 156.21 112.395) (width 0.254) (layer F.Cu) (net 46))
 (segment (start 156.21 112.395) (end 156.21 116.76) (width 0.254) (layer F.Cu) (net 46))
 (segment (start 151.765 102.49) (end 151.765 109.22) (width 0.254) (layer F.Cu) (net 47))
 (segment (start 151.765 109.22) (end 153.67 111.125) (width 0.254) (layer F.Cu) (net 47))
 (segment (start 153.67 111.125) (end 153.67 116.76) (width 0.254) (layer F.Cu) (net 47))
 (segment (start 150.495 102.49) (end 150.495 109.22) (width 0.254) (layer F.Cu) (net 48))
 (segment (start 150.495 109.22) (end 151.13 109.855) (width 0.254) (layer F.Cu) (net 48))
 (segment (start 151.13 109.855) (end 151.13 116.76) (width 0.254) (layer F.Cu) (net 48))
 (segment (start 149.225 102.49) (end 149.225 109.22) (width 0.254) (layer F.Cu) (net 49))
 (segment (start 149.225 109.22) (end 148.59 109.855) (width 0.254) (layer F.Cu) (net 49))
 (segment (start 148.59 109.855) (end 148.59 116.76) (width 0.254) (layer F.Cu) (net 49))
 (segment (start 147.955 102.49) (end 147.955 109.22) (width 0.254) (layer F.Cu) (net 50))
 (segment (start 147.955 109.22) (end 146.05 111.125) (width 0.254) (layer F.Cu) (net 50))
 (segment (start 146.05 111.125) (end 146.05 116.76) (width 0.254) (layer F.Cu) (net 50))
 (segment (start 146.685 102.49) (end 146.685 109.22) (width 0.254) (layer F.Cu) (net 51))
 (segment (start 146.685 109.22) (end 143.51 112.395) (width 0.254) (layer F.Cu) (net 51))
 (segment (start 143.51 112.395) (end 143.51 116.76) (width 0.254) (layer F.Cu) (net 51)))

